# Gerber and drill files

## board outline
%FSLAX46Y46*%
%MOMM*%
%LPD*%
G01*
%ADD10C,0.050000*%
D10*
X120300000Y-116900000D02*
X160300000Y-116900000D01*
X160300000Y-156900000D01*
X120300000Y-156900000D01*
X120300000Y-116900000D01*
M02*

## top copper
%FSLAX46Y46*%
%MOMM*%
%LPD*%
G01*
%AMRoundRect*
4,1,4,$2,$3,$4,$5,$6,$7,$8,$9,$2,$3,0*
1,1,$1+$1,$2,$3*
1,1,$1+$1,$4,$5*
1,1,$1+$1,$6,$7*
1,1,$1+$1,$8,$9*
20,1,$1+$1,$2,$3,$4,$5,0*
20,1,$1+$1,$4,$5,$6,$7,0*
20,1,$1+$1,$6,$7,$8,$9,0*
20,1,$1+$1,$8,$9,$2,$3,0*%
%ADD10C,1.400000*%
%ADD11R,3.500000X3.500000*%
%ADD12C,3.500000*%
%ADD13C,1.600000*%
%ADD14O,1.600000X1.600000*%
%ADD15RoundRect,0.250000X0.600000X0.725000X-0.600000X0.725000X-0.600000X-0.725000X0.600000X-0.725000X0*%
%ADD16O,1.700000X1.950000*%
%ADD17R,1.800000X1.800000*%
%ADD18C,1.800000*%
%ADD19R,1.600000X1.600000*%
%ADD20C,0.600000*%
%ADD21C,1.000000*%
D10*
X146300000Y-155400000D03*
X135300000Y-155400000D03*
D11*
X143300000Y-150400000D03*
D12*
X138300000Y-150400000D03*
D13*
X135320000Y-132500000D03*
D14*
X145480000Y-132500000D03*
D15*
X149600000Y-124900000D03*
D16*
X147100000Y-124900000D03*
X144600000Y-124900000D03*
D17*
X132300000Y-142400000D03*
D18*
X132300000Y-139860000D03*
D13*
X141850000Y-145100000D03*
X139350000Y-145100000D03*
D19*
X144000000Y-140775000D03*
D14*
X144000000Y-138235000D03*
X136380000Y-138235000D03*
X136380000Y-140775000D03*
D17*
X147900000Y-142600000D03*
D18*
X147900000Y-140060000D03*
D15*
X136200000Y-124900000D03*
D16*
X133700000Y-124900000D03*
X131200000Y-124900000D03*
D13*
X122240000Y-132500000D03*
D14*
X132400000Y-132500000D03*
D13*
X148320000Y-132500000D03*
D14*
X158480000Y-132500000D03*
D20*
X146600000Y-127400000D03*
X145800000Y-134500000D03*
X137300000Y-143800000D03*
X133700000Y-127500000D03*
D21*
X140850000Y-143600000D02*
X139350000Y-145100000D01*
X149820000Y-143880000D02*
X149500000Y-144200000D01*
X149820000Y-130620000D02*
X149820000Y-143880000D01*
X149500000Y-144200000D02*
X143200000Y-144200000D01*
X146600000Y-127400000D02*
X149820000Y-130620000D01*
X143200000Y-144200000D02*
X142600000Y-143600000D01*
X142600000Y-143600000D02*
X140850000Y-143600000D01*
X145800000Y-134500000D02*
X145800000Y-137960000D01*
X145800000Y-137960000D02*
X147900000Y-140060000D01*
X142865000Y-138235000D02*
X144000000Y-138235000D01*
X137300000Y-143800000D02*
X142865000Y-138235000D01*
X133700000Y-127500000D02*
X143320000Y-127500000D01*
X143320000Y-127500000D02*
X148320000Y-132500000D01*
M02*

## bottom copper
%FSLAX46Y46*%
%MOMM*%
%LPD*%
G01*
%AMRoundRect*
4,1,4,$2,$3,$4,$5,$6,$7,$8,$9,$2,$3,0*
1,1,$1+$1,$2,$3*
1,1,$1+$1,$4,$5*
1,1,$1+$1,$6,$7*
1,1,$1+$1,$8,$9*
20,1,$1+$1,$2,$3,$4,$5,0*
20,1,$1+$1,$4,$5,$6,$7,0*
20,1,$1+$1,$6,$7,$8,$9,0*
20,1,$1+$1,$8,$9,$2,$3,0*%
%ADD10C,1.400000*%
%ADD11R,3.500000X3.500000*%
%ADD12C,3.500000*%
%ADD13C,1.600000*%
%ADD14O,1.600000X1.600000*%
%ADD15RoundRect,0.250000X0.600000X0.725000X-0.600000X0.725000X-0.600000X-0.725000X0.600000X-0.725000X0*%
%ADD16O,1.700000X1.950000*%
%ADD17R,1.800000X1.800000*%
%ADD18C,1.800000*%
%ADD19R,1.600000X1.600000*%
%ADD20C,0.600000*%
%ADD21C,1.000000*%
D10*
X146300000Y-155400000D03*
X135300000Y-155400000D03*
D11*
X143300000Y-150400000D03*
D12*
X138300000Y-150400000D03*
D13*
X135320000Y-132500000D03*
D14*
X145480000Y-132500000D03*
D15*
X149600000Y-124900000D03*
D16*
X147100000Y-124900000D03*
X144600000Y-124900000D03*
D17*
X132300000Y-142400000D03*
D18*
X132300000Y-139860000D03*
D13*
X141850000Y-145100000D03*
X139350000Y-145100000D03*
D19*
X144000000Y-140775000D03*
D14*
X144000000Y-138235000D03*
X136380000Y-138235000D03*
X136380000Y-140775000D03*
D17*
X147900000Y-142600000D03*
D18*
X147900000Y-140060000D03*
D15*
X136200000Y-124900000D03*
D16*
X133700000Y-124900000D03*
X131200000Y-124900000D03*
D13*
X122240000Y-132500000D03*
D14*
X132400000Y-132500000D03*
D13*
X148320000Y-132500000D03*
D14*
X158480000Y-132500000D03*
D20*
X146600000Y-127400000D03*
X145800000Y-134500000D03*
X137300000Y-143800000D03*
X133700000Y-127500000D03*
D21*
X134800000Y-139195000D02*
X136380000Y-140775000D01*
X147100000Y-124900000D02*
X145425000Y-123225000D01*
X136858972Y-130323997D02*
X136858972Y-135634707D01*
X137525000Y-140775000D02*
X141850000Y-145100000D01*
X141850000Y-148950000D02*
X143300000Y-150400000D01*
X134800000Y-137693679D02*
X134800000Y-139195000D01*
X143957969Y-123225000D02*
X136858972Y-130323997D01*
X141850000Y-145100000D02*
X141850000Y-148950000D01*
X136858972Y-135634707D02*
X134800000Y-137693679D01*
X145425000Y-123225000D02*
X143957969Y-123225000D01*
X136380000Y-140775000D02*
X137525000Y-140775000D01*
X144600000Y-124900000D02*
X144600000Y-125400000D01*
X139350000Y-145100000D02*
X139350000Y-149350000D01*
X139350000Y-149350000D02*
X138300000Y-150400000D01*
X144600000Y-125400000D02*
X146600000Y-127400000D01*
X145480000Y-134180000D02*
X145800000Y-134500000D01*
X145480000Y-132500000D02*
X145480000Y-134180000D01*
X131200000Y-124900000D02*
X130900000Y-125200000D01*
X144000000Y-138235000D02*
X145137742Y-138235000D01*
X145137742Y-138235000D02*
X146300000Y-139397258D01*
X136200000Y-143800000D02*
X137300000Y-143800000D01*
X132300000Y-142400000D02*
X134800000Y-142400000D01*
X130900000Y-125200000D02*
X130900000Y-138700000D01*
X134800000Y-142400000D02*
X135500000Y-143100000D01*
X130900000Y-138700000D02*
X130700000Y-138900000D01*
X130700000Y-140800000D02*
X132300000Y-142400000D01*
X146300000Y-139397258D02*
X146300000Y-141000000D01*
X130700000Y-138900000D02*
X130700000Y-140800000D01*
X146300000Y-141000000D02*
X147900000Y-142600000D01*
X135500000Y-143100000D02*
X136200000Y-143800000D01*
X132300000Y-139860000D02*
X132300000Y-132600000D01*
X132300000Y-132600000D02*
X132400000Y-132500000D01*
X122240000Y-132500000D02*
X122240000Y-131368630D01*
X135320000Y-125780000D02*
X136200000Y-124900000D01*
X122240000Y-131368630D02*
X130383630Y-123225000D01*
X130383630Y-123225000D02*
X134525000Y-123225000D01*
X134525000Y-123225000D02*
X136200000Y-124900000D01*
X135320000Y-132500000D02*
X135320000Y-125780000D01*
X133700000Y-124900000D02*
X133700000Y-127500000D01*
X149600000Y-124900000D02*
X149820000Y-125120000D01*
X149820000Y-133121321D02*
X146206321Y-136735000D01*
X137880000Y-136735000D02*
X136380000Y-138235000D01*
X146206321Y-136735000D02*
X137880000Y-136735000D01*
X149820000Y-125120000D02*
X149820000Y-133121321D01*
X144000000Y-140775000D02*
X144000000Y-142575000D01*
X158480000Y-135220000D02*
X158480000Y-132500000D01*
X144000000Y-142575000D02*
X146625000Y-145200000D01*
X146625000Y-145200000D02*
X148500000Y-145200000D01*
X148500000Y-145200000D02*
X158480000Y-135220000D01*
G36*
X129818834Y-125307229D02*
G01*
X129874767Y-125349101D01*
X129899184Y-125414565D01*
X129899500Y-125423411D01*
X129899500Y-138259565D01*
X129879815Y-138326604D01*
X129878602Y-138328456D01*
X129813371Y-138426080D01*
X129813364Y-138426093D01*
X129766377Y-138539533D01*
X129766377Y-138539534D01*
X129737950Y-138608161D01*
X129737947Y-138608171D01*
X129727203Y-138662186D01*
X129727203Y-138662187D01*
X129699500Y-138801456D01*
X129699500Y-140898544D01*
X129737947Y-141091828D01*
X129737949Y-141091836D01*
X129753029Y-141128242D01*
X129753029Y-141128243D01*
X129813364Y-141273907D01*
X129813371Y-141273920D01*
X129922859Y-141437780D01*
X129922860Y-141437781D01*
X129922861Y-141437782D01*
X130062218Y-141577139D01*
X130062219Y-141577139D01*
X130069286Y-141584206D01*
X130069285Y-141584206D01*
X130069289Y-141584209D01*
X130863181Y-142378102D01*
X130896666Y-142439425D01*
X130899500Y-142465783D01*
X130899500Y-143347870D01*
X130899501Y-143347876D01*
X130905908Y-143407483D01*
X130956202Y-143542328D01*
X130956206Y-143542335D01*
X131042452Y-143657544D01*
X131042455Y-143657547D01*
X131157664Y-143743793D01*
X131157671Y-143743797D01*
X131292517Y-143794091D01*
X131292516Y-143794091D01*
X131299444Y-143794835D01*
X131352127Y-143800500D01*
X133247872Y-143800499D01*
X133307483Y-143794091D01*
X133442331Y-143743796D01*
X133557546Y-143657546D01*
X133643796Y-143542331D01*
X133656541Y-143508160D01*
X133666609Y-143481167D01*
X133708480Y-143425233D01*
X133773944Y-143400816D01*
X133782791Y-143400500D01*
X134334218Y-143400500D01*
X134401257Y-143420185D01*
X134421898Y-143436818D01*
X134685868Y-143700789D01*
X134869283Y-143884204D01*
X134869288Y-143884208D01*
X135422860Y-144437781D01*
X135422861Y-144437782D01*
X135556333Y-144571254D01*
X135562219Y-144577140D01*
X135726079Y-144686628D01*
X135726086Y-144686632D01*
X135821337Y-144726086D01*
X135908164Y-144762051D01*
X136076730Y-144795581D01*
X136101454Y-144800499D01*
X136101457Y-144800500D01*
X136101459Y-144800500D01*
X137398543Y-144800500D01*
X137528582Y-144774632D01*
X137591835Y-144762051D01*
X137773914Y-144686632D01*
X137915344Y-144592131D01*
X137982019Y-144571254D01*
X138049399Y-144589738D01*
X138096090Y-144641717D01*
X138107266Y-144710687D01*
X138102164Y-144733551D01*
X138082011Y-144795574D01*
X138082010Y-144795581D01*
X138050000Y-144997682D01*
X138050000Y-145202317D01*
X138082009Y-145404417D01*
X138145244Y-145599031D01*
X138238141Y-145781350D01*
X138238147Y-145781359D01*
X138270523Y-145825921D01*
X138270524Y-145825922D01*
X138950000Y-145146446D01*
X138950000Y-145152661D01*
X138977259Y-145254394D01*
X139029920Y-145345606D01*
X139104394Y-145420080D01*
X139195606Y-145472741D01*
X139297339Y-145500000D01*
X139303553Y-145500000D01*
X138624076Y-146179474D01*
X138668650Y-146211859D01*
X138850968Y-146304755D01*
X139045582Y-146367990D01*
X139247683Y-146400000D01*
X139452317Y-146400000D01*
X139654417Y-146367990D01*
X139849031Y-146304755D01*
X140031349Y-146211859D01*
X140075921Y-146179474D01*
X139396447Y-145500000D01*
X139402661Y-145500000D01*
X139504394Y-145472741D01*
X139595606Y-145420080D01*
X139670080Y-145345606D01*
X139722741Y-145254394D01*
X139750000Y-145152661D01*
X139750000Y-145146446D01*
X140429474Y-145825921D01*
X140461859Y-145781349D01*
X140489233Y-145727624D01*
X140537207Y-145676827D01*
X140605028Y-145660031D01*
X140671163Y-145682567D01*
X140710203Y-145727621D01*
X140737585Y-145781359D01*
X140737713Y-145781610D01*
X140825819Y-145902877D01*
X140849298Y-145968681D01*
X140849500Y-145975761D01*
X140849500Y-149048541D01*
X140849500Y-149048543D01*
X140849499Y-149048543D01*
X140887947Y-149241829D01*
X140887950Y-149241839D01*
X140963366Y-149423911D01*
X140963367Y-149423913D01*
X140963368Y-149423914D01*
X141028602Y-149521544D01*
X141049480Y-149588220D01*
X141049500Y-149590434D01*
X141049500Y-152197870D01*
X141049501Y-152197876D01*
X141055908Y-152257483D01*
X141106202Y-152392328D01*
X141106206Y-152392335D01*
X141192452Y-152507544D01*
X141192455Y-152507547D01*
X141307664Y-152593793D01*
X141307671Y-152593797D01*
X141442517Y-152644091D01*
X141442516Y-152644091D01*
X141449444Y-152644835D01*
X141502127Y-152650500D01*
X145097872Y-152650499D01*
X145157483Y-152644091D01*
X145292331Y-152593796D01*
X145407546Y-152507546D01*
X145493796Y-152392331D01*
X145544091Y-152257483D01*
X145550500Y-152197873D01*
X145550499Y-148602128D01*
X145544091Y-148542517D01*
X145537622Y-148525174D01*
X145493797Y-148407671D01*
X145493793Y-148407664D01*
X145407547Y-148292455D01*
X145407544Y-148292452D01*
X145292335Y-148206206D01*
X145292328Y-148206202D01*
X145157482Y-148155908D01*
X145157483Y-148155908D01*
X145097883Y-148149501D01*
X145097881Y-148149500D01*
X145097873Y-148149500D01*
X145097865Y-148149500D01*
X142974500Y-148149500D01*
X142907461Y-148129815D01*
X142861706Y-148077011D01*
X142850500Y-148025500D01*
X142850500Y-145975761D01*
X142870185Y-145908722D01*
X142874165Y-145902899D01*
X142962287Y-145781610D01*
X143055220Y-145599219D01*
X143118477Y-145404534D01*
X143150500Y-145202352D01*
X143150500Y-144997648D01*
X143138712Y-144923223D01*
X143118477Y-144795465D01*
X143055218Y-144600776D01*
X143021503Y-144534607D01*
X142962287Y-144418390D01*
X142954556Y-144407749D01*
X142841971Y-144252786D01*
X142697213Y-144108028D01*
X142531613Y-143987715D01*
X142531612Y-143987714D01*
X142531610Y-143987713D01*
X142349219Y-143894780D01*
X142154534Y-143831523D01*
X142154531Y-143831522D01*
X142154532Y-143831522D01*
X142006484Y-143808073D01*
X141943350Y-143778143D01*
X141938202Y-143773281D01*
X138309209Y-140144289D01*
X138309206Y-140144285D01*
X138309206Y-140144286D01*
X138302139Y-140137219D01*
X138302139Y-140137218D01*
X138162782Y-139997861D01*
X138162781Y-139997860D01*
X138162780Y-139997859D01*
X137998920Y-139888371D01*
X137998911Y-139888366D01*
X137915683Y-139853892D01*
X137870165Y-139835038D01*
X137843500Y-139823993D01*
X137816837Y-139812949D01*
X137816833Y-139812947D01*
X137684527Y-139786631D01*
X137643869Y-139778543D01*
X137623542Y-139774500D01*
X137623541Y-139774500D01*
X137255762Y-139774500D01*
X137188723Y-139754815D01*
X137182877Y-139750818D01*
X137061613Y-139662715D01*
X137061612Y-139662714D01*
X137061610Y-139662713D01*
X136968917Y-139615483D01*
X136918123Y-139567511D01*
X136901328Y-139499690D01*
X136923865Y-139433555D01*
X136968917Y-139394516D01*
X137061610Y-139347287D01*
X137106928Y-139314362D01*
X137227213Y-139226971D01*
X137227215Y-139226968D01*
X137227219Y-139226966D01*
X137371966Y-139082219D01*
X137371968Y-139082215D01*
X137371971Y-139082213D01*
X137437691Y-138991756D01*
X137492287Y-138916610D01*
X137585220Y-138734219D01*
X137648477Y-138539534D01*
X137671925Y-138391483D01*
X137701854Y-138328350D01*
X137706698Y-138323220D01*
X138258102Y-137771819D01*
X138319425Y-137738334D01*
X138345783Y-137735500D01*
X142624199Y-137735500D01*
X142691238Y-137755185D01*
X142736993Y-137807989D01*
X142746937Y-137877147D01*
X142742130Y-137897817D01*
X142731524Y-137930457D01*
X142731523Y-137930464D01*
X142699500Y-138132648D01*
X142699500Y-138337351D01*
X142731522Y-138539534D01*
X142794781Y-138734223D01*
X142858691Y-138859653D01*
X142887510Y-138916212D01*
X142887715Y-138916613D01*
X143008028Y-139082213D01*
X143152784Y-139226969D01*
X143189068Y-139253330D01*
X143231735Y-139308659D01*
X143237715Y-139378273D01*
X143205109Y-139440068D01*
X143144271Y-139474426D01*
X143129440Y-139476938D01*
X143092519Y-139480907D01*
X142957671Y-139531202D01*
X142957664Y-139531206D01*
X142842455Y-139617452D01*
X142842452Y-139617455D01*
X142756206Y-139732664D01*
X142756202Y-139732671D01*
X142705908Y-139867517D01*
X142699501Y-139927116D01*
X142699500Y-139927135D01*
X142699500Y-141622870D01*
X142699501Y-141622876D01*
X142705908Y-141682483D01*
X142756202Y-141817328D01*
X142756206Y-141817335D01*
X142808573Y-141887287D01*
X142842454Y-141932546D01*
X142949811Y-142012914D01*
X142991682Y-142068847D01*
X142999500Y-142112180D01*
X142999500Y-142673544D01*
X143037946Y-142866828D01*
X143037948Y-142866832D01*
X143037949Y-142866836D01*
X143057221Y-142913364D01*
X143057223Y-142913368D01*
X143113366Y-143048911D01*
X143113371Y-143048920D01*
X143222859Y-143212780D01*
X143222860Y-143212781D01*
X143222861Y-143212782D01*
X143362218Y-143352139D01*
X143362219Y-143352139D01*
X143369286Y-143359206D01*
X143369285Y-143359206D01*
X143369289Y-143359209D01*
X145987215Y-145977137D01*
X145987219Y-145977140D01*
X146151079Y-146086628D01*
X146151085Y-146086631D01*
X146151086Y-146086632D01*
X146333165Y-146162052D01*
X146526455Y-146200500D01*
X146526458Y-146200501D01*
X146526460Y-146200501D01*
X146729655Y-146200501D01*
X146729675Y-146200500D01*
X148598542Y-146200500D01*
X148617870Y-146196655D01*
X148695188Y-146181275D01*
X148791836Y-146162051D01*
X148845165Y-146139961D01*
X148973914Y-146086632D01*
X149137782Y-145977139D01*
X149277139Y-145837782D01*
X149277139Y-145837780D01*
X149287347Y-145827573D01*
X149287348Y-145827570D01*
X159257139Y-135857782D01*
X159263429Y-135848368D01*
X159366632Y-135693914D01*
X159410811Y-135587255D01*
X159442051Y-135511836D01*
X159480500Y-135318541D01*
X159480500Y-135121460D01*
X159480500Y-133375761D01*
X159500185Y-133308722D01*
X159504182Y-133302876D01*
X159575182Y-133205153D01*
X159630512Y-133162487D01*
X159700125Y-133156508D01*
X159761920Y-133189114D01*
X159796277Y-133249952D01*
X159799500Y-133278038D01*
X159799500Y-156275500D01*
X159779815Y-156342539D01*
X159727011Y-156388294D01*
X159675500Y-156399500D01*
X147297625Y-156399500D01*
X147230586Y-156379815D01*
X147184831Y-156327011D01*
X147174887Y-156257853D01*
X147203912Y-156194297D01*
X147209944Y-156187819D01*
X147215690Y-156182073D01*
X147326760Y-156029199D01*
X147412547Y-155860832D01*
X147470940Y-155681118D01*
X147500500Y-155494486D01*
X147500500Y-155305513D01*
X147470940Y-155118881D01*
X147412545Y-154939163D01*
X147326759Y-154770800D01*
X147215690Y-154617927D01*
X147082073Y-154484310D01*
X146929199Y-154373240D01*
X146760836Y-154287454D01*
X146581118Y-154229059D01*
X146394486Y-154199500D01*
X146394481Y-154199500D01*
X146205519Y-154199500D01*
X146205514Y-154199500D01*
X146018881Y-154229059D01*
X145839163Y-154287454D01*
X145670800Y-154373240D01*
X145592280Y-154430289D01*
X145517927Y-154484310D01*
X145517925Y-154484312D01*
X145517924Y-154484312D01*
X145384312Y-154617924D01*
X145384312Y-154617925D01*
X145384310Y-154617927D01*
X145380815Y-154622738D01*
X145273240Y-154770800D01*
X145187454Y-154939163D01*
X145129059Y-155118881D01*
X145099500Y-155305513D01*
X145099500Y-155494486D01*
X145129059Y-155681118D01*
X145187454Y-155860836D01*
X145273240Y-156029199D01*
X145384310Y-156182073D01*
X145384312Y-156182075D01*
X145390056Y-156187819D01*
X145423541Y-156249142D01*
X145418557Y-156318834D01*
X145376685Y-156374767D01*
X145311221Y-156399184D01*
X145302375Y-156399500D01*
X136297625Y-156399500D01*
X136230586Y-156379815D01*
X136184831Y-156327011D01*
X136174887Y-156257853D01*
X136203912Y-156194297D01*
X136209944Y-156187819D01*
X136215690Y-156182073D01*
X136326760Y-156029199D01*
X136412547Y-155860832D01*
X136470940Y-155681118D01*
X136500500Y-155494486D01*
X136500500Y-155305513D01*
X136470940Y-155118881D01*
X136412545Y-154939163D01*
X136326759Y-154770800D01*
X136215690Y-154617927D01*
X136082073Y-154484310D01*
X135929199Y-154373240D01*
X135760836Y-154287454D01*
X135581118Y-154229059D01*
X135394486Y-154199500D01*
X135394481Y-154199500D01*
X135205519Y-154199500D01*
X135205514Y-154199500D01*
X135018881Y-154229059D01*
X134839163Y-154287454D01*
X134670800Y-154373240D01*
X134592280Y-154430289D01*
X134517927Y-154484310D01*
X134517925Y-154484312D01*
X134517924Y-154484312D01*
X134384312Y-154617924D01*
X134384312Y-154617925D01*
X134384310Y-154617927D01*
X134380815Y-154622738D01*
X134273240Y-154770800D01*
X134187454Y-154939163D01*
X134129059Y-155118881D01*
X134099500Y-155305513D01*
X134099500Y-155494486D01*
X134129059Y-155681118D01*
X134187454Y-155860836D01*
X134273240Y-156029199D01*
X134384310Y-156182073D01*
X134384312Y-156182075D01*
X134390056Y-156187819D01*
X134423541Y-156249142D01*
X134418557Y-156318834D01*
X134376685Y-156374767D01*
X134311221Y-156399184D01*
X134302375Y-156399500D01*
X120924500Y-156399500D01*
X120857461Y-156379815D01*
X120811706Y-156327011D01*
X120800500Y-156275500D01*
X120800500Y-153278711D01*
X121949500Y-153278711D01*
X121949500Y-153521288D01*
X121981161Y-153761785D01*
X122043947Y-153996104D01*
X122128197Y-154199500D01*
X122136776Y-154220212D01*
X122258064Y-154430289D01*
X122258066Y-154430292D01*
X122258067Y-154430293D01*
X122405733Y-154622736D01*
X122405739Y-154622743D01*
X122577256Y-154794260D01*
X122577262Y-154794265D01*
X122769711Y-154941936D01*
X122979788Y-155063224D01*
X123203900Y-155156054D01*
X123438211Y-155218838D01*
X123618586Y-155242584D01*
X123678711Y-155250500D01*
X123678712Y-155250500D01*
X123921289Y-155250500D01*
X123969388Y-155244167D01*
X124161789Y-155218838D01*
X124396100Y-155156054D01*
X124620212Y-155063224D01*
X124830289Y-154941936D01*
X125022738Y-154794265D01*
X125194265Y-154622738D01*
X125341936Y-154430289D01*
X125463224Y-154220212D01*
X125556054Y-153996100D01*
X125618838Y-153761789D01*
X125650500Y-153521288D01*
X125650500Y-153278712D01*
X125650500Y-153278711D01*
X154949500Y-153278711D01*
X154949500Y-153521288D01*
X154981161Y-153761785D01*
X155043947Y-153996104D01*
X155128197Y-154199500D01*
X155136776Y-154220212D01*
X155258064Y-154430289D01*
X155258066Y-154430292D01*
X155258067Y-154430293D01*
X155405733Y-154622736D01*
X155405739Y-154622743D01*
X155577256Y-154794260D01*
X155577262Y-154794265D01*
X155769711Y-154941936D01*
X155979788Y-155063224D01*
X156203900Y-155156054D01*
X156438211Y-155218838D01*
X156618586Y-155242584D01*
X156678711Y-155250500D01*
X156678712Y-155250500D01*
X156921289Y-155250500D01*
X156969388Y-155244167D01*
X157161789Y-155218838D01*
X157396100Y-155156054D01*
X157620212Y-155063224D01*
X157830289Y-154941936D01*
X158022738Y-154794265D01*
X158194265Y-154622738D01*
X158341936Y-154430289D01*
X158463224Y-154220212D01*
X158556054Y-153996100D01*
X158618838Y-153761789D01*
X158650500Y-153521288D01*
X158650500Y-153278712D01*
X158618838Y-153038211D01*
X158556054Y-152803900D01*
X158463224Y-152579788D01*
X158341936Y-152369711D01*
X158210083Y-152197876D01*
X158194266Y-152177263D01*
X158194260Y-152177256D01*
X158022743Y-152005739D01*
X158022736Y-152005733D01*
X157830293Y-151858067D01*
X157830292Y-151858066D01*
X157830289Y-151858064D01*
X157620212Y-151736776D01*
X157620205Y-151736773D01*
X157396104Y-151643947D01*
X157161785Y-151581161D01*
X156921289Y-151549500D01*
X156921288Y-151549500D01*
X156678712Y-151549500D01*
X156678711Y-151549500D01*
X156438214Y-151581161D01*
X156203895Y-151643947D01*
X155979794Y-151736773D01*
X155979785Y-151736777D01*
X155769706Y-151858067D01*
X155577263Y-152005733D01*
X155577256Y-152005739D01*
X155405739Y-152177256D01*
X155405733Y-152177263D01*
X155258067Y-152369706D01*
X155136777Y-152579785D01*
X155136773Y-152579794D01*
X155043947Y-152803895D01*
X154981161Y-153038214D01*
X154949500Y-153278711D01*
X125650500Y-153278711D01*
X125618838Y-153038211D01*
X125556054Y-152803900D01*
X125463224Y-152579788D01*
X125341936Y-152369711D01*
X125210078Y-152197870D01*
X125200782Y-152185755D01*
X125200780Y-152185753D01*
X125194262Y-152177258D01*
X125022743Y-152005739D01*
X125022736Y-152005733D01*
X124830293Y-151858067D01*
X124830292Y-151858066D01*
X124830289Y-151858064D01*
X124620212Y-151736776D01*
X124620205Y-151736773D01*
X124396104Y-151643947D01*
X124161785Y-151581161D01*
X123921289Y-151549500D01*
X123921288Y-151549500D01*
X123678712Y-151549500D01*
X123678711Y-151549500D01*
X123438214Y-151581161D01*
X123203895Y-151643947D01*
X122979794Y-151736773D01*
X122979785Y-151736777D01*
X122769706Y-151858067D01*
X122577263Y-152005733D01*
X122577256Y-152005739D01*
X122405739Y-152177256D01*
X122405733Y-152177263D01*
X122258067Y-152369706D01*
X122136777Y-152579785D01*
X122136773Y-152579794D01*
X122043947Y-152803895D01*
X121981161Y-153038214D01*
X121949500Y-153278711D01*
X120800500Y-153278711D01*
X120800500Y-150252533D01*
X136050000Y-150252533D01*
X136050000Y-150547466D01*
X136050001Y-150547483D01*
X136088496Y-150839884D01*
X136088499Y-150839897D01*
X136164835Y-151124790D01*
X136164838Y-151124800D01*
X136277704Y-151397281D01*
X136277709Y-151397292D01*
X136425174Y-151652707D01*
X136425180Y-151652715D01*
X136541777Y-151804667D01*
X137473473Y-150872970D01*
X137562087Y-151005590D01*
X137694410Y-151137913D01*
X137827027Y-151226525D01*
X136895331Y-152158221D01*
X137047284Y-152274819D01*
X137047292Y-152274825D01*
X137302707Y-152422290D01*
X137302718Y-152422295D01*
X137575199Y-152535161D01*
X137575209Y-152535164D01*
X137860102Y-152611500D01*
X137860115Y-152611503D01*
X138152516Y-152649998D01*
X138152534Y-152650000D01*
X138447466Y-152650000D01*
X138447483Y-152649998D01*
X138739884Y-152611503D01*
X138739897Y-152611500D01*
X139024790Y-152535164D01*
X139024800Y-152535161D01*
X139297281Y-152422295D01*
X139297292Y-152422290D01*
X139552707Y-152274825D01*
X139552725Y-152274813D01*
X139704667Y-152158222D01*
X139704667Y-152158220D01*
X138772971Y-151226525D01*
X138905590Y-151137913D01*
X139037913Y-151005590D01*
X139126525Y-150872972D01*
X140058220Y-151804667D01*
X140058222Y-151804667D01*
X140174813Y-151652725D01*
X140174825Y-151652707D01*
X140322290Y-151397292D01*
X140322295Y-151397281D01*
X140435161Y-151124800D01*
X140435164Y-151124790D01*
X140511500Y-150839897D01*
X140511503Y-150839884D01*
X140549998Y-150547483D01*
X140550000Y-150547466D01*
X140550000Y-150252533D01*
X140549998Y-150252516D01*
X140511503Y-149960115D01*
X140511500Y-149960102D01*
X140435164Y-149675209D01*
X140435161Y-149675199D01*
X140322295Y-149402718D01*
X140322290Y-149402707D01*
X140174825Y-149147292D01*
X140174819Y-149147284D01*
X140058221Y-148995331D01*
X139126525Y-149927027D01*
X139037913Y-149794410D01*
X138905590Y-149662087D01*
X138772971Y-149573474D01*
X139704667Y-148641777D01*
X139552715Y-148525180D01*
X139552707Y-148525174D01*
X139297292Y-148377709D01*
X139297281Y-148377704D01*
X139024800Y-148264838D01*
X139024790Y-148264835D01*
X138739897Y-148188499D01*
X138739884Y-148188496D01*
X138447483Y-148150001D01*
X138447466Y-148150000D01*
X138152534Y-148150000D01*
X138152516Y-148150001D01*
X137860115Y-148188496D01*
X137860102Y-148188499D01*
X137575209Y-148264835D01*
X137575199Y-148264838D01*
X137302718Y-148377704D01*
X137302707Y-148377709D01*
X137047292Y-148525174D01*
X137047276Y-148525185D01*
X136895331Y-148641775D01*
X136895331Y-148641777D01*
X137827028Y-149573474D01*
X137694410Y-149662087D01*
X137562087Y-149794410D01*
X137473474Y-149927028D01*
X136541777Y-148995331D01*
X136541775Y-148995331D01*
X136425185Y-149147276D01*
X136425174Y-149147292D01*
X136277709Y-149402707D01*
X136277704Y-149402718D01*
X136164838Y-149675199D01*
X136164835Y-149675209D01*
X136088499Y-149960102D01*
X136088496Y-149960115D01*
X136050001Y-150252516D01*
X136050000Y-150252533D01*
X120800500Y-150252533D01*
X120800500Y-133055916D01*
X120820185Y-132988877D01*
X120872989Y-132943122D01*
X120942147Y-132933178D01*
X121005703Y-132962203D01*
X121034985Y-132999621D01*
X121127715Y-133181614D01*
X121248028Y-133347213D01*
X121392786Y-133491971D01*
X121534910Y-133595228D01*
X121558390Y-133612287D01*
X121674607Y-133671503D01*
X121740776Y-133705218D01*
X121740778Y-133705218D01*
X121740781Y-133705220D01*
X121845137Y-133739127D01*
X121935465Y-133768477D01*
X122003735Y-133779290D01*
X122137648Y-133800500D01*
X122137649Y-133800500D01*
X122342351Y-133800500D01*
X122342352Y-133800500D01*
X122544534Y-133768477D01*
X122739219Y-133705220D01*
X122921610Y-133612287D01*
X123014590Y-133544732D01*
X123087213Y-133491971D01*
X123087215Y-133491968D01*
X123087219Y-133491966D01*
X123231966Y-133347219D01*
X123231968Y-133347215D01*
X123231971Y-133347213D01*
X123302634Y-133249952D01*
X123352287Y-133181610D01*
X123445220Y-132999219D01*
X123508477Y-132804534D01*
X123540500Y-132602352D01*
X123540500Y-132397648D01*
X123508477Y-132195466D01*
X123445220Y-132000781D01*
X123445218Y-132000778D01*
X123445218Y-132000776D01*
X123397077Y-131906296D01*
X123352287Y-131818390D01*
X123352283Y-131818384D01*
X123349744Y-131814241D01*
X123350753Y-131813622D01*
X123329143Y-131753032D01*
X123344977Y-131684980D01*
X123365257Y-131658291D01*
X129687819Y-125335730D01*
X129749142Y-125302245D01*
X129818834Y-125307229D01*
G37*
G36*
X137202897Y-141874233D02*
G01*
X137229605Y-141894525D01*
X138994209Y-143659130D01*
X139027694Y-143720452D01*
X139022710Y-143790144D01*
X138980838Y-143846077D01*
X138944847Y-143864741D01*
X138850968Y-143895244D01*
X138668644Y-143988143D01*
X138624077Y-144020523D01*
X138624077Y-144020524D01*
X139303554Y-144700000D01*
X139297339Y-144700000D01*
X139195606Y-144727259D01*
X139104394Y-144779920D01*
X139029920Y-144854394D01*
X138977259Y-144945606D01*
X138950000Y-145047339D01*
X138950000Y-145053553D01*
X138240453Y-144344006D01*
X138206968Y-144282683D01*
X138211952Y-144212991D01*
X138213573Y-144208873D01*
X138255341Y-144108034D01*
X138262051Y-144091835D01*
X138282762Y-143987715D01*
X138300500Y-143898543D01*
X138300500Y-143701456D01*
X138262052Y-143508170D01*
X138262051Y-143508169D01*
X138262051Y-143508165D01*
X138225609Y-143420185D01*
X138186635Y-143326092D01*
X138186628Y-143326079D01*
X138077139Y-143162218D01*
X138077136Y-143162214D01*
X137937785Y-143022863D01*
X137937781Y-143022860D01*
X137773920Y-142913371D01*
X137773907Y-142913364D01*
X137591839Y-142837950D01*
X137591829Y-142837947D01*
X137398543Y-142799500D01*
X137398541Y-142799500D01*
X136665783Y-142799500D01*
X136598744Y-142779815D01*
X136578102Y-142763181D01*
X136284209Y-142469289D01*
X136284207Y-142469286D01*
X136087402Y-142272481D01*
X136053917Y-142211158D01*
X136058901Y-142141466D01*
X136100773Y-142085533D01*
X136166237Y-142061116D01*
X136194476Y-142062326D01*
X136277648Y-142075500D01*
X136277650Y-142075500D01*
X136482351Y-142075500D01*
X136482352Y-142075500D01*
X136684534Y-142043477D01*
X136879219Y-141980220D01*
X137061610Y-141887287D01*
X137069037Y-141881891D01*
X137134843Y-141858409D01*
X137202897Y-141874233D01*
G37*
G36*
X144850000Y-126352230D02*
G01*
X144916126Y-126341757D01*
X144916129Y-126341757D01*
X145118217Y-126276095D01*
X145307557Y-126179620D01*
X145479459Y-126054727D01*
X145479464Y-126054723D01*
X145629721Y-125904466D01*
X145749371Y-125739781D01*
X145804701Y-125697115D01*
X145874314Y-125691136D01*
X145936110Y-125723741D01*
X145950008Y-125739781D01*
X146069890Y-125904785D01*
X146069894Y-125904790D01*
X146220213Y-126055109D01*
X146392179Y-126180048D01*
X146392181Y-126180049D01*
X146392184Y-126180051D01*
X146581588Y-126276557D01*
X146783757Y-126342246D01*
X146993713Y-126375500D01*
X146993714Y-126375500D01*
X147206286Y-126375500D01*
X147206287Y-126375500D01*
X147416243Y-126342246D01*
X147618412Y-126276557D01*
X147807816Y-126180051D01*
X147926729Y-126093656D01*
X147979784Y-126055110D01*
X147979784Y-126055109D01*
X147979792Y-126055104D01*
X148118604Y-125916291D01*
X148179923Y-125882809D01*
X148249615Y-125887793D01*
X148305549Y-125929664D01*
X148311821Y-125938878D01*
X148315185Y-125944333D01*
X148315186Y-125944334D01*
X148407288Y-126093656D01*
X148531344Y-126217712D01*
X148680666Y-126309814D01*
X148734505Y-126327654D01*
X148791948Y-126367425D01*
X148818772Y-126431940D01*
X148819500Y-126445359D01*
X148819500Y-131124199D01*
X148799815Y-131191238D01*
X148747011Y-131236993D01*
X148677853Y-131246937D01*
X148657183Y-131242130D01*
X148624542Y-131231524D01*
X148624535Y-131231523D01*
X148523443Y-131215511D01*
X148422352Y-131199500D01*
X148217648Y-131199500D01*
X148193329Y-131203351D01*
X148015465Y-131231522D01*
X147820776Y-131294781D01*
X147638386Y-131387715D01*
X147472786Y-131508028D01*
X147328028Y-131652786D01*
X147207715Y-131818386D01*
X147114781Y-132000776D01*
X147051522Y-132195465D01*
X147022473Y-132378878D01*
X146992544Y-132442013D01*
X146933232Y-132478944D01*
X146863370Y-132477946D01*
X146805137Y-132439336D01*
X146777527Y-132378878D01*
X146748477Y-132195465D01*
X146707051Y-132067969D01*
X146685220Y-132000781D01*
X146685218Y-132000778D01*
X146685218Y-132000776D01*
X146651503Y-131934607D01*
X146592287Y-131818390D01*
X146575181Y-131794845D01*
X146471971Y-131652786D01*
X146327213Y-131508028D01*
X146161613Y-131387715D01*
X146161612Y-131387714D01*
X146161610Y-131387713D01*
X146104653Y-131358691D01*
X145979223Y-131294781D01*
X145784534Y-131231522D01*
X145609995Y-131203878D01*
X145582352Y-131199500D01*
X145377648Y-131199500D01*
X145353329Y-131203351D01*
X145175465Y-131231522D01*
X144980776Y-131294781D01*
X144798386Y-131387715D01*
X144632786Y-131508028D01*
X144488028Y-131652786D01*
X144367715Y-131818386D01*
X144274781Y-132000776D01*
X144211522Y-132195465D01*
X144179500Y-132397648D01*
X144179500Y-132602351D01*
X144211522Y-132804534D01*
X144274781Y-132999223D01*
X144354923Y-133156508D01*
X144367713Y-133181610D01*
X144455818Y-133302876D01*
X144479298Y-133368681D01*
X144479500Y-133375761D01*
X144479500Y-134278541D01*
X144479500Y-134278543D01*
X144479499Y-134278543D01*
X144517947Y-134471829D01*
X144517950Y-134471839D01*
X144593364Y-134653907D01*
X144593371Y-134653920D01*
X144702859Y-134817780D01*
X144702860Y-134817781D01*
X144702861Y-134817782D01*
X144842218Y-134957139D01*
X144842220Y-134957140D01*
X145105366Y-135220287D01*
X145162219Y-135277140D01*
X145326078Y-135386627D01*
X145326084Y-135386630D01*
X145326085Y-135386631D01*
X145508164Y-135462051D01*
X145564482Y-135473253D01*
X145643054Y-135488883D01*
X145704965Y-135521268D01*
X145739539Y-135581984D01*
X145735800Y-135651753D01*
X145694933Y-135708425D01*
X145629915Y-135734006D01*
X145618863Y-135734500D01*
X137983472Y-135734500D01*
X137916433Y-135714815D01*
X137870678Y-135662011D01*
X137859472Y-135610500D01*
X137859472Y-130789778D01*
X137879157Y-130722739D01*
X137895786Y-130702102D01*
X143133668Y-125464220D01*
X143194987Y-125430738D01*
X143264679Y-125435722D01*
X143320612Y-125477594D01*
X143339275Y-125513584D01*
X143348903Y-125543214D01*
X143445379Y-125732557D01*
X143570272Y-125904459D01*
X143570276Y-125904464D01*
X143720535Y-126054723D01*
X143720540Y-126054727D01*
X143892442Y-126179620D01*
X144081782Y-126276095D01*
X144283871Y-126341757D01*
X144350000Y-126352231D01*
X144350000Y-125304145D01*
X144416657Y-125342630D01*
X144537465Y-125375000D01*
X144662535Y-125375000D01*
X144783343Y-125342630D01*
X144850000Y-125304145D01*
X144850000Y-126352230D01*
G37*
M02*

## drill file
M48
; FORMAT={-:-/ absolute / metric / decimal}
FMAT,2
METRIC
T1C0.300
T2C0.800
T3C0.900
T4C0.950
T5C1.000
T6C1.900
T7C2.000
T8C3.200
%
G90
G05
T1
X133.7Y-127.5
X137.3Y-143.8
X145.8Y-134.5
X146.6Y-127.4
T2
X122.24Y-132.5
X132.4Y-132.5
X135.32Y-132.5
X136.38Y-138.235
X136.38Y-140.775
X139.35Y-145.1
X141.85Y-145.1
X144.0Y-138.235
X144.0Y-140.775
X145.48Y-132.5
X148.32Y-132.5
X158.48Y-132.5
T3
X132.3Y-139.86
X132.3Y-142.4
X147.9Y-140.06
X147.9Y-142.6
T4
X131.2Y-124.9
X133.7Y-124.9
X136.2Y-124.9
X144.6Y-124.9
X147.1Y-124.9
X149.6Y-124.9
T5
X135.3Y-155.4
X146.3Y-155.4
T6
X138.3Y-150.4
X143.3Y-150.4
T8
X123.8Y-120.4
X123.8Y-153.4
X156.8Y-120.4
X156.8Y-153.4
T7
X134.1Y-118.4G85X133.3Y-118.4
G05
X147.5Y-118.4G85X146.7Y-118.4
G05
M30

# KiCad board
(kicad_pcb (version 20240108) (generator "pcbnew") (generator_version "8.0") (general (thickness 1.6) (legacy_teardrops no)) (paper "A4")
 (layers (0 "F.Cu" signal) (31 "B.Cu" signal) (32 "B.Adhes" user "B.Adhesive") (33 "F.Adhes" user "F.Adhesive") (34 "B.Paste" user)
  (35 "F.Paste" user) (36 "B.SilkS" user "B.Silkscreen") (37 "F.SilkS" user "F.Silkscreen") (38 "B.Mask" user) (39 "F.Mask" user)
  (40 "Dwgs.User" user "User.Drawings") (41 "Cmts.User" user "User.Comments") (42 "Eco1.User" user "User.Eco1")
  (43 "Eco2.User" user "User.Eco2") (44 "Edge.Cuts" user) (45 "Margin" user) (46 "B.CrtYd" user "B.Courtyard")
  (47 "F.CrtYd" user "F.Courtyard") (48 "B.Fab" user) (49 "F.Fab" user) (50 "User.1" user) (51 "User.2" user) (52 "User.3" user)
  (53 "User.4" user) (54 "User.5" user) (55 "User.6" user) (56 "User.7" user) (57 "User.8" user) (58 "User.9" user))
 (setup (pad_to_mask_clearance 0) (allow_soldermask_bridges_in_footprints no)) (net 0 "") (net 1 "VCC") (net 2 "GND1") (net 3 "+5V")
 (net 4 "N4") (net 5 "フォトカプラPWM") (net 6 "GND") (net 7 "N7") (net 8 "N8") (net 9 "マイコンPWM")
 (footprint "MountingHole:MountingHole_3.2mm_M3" (layer "F.Cu") (at 123.8 153.4)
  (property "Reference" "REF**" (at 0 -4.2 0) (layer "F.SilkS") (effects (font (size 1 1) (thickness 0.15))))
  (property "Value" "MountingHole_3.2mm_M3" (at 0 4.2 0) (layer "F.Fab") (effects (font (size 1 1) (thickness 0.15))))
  (pad "" np_thru_hole circle (at 0 0) (size 3.2 3.2) (drill 3.2) (layers "*.Cu" "*.Mask")))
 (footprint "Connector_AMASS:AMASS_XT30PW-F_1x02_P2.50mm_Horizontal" (layer "F.Cu") (at 143.3 150.4 180)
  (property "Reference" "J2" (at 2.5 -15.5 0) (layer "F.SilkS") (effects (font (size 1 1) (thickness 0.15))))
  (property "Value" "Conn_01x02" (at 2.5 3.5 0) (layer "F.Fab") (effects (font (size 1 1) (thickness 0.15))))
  (pad "" thru_hole circle (at -3 -5 270) (size 1.4 1.4) (drill 1) (layers "*.Cu" "*.Mask") (remove_unused_layers no))
  (pad "" thru_hole circle (at 8 -5 180) (size 1.4 1.4) (drill 1) (layers "*.Cu" "*.Mask") (remove_unused_layers no))
  (pad "1" thru_hole rect (at 0 0 180) (size 3.5 3.5) (drill 1.9) (layers "*.Cu" "*.Mask") (remove_unused_layers no) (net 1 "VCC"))
  (pad "2" thru_hole circle (at 5 0 180) (size 3.5 3.5) (drill 1.9) (layers "*.Cu" "*.Mask") (remove_unused_layers no) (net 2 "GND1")))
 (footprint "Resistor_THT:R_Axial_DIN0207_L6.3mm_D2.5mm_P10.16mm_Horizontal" (layer "F.Cu") (at 135.32 132.5)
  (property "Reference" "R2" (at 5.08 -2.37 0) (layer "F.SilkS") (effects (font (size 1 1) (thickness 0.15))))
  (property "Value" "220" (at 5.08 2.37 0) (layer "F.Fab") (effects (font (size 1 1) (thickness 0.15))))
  (pad "1" thru_hole circle (at 0 0) (size 1.6 1.6) (drill 0.8) (layers "*.Cu" "*.Mask") (remove_unused_layers no) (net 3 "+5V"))
  (pad "2" thru_hole oval (at 10.16 0) (size 1.6 1.6) (drill 0.8) (layers "*.Cu" "*.Mask") (remove_unused_layers no) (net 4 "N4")))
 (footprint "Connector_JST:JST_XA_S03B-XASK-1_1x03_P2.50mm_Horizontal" (layer "F.Cu") (at 149.6 124.9 180)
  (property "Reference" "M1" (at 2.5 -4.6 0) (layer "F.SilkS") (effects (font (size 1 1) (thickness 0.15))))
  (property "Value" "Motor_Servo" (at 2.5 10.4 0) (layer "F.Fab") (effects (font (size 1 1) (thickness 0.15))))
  (pad "" np_thru_hole oval (at 2.5 6.5 180) (size 2.8 2) (drill oval 2.8 2) (layers "*.Cu" "*.Mask"))
  (pad "1" thru_hole roundrect (at 0 0 180) (size 1.7 1.95) (drill 0.95) (layers "*.Cu" "*.Mask") (remove_unused_layers no)
   (roundrect_rratio 0.147059) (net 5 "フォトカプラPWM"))
  (pad "2" thru_hole oval (at 2.5 0 180) (size 1.7 1.95) (drill 0.95) (layers "*.Cu" "*.Mask") (remove_unused_layers no) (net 1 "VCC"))
  (pad "3" thru_hole oval (at 5 0 180) (size 1.7 1.95) (drill 0.95) (layers "*.Cu" "*.Mask") (remove_unused_layers no) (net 2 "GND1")))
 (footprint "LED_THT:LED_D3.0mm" (layer "F.Cu") (at 132.3 142.4 90)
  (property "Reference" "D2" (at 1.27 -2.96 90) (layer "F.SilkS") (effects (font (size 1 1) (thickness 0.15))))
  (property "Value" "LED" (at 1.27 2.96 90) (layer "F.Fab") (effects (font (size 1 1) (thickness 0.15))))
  (pad "1" thru_hole rect (at 0 0 90) (size 1.8 1.8) (drill 0.9) (layers "*.Cu" "*.Mask") (remove_unused_layers no) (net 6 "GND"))
  (pad "2" thru_hole circle (at 2.54 0 90) (size 1.8 1.8) (drill 0.9) (layers "*.Cu" "*.Mask") (remove_unused_layers no) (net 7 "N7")))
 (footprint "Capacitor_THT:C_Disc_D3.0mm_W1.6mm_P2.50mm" (layer "F.Cu") (at 141.85 145.1 180)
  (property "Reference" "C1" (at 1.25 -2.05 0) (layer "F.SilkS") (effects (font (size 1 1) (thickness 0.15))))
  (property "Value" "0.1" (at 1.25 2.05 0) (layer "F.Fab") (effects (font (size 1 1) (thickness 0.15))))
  (pad "1" thru_hole circle (at 0 0 180) (size 1.6 1.6) (drill 0.8) (layers "*.Cu" "*.Mask") (remove_unused_layers no) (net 1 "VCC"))
  (pad "2" thru_hole circle (at 2.5 0 180) (size 1.6 1.6) (drill 0.8) (layers "*.Cu" "*.Mask") (remove_unused_layers no) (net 2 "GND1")))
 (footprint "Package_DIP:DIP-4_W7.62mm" (layer "F.Cu") (at 144 140.775 180)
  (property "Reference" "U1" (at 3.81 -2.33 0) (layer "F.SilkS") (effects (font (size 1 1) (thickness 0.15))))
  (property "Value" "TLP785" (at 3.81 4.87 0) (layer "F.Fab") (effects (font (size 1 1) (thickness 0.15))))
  (pad "1" thru_hole rect (at 0 0 180) (size 1.6 1.6) (drill 0.8) (layers "*.Cu" "*.Mask") (remove_unused_layers no) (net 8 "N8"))
  (pad "2" thru_hole oval (at 0 2.54 180) (size 1.6 1.6) (drill 0.8) (layers "*.Cu" "*.Mask") (remove_unused_layers no) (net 6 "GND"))
  (pad "3" thru_hole oval (at 7.62 2.54 180) (size 1.6 1.6) (drill 0.8) (layers "*.Cu" "*.Mask") (remove_unused_layers no)
   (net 5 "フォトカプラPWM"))
  (pad "4" thru_hole oval (at 7.62 0 180) (size 1.6 1.6) (drill 0.8) (layers "*.Cu" "*.Mask") (remove_unused_layers no) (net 1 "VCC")))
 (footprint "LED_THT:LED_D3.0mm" (layer "F.Cu") (at 147.9 142.6 90)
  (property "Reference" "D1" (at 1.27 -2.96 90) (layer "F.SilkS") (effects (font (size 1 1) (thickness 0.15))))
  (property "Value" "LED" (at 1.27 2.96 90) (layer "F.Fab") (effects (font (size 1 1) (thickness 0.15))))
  (pad "1" thru_hole rect (at 0 0 90) (size 1.8 1.8) (drill 0.9) (layers "*.Cu" "*.Mask") (remove_unused_layers no) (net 6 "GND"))
  (pad "2" thru_hole circle (at 2.54 0 90) (size 1.8 1.8) (drill 0.9) (layers "*.Cu" "*.Mask") (remove_unused_layers no) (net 4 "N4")))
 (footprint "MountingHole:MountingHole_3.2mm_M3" (layer "F.Cu") (at 156.8 153.4)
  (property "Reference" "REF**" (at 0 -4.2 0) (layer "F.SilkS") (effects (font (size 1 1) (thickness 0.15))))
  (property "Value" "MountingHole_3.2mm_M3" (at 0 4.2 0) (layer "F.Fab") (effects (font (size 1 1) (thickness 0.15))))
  (pad "" np_thru_hole circle (at 0 0) (size 3.2 3.2) (drill 3.2) (layers "*.Cu" "*.Mask")))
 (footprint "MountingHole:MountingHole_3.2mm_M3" (layer "F.Cu") (at 156.8 120.4)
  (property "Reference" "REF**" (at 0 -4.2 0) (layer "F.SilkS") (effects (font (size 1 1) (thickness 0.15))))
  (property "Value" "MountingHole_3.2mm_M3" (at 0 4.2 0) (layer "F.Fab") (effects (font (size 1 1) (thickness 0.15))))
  (pad "" np_thru_hole circle (at 0 0) (size 3.2 3.2) (drill 3.2) (layers "*.Cu" "*.Mask")))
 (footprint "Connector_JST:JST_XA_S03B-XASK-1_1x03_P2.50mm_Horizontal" (layer "F.Cu") (at 136.2 124.9 180)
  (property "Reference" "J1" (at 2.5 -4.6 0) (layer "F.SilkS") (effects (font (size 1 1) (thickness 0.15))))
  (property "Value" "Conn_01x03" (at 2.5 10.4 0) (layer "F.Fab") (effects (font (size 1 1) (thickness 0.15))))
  (pad "" np_thru_hole oval (at 2.5 6.5 180) (size 2.8 2) (drill oval 2.8 2) (layers "*.Cu" "*.Mask"))
  (pad "1" thru_hole roundrect (at 0 0 180) (size 1.7 1.95) (drill 0.95) (layers "*.Cu" "*.Mask") (remove_unused_layers no)
   (roundrect_rratio 0.147059) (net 3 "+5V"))
  (pad "2" thru_hole oval (at 2.5 0 180) (size 1.7 1.95) (drill 0.95) (layers "*.Cu" "*.Mask") (remove_unused_layers no) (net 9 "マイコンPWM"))
  (pad "3" thru_hole oval (at 5 0 180) (size 1.7 1.95) (drill 0.95) (layers "*.Cu" "*.Mask") (remove_unused_layers no) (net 6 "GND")))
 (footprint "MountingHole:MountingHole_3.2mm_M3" (layer "F.Cu") (at 123.8 120.4)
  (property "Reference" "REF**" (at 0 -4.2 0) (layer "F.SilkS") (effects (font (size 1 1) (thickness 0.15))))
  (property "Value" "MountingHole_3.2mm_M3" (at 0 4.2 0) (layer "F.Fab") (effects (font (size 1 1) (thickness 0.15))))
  (pad "" np_thru_hole circle (at 0 0) (size 3.2 3.2) (drill 3.2) (layers "*.Cu" "*.Mask")))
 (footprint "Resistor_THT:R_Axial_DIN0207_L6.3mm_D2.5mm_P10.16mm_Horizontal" (layer "F.Cu") (at 122.24 132.5)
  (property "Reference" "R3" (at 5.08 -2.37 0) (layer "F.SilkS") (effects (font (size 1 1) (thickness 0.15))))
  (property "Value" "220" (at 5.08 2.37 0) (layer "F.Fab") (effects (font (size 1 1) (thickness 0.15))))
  (pad "1" thru_hole circle (at 0 0) (size 1.6 1.6) (drill 0.8) (layers "*.Cu" "*.Mask") (remove_unused_layers no) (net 3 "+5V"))
  (pad "2" thru_hole oval (at 10.16 0) (size 1.6 1.6) (drill 0.8) (layers "*.Cu" "*.Mask") (remove_unused_layers no) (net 7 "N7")))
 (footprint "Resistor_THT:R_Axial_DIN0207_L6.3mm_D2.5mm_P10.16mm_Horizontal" (layer "F.Cu") (at 148.32 132.5)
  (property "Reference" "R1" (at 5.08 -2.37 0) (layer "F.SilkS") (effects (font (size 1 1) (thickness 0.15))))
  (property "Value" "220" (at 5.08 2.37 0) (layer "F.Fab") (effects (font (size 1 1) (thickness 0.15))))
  (pad "1" thru_hole circle (at 0 0) (size 1.6 1.6) (drill 0.8) (layers "*.Cu" "*.Mask") (remove_unused_layers no) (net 9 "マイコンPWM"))
  (pad "2" thru_hole oval (at 10.16 0) (size 1.6 1.6) (drill 0.8) (layers "*.Cu" "*.Mask") (remove_unused_layers no) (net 8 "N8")))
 (gr_rect (start 120.3 116.9) (end 160.3 156.9) (stroke (width 0.05) (type default)) (fill none) (layer "Edge.Cuts"))
 (segment (start 134.8 139.195) (end 136.38 140.775) (width 1) (layer "B.Cu") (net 1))
 (segment (start 147.1 124.9) (end 145.425 123.225) (width 1) (layer "B.Cu") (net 1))
 (segment (start 136.858972 130.323997) (end 136.858972 135.634707) (width 1) (layer "B.Cu") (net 1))
 (segment (start 137.525 140.775) (end 141.85 145.1) (width 1) (layer "B.Cu") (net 1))
 (segment (start 141.85 148.95) (end 143.3 150.4) (width 1) (layer "B.Cu") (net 1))
 (segment (start 134.8 137.693679) (end 134.8 139.195) (width 1) (layer "B.Cu") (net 1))
 (segment (start 143.957969 123.225) (end 136.858972 130.323997) (width 1) (layer "B.Cu") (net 1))
 (segment (start 141.85 145.1) (end 141.85 148.95) (width 1) (layer "B.Cu") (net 1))
 (segment (start 136.858972 135.634707) (end 134.8 137.693679) (width 1) (layer "B.Cu") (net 1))
 (segment (start 145.425 123.225) (end 143.957969 123.225) (width 1) (layer "B.Cu") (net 1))
 (segment (start 136.38 140.775) (end 137.525 140.775) (width 1) (layer "B.Cu") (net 1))
 (segment (start 140.85 143.6) (end 139.35 145.1) (width 1) (layer "F.Cu") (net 2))
 (segment (start 149.82 143.88) (end 149.5 144.2) (width 1) (layer "F.Cu") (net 2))
 (segment (start 149.82 130.62) (end 149.82 143.88) (width 1) (layer "F.Cu") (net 2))
 (segment (start 149.5 144.2) (end 143.2 144.2) (width 1) (layer "F.Cu") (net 2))
 (segment (start 146.6 127.4) (end 149.82 130.62) (width 1) (layer "F.Cu") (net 2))
 (segment (start 143.2 144.2) (end 142.6 143.6) (width 1) (layer "F.Cu") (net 2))
 (segment (start 142.6 143.6) (end 140.85 143.6) (width 1) (layer "F.Cu") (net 2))
 (via (at 146.6 127.4) (size 0.6) (drill 0.3) (layers "F.Cu" "B.Cu") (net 2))
 (segment (start 144.6 124.9) (end 144.6 125.4) (width 1) (layer "B.Cu") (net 2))
 (segment (start 139.35 145.1) (end 139.35 149.35) (width 1) (layer "B.Cu") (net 2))
 (segment (start 139.35 149.35) (end 138.3 150.4) (width 1) (layer "B.Cu") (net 2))
 (segment (start 144.6 125.4) (end 146.6 127.4) (width 1) (layer "B.Cu") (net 2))
 (segment (start 145.8 134.5) (end 145.8 137.96) (width 1) (layer "F.Cu") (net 4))
 (segment (start 145.8 137.96) (end 147.9 140.06) (width 1) (layer "F.Cu") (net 4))
 (via (at 145.8 134.5) (size 0.6) (drill 0.3) (layers "F.Cu" "B.Cu") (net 4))
 (segment (start 145.48 134.18) (end 145.8 134.5) (width 1) (layer "B.Cu") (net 4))
 (segment (start 145.48 132.5) (end 145.48 134.18) (width 1) (layer "B.Cu") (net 4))
 (segment (start 142.865 138.235) (end 144 138.235) (width 1) (layer "F.Cu") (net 6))
 (segment (start 137.3 143.8) (end 142.865 138.235) (width 1) (layer "F.Cu") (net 6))
 (via (at 137.3 143.8) (size 0.6) (drill 0.3) (layers "F.Cu" "B.Cu") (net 6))
 (segment (start 131.2 124.9) (end 130.9 125.2) (width 1) (layer "B.Cu") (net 6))
 (segment (start 144 138.235) (end 145.137742 138.235) (width 1) (layer "B.Cu") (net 6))
 (segment (start 145.137742 138.235) (end 146.3 139.397258) (width 1) (layer "B.Cu") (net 6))
 (segment (start 136.2 143.8) (end 137.3 143.8) (width 1) (layer "B.Cu") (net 6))
 (segment (start 132.3 142.4) (end 134.8 142.4) (width 1) (layer "B.Cu") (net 6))
 (segment (start 130.9 125.2) (end 130.9 138.7) (width 1) (layer "B.Cu") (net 6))
 (segment (start 134.8 142.4) (end 135.5 143.1) (width 1) (layer "B.Cu") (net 6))
 (segment (start 130.9 138.7) (end 130.7 138.9) (width 1) (layer "B.Cu") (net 6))
 (segment (start 130.7 140.8) (end 132.3 142.4) (width 1) (layer "B.Cu") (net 6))
 (segment (start 146.3 139.397258) (end 146.3 141) (width 1) (layer "B.Cu") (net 6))
 (segment (start 130.7 138.9) (end 130.7 140.8) (width 1) (layer "B.Cu") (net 6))
 (segment (start 146.3 141) (end 147.9 142.6) (width 1) (layer "B.Cu") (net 6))
 (segment (start 135.5 143.1) (end 136.2 143.8) (width 1) (layer "B.Cu") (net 6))
 (segment (start 132.3 139.86) (end 132.3 132.6) (width 1) (layer "B.Cu") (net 7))
 (segment (start 132.3 132.6) (end 132.4 132.5) (width 1) (layer "B.Cu") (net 7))
 (segment (start 122.24 132.5) (end 122.24 131.36863) (width 1) (layer "B.Cu") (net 3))
 (segment (start 135.32 125.78) (end 136.2 124.9) (width 1) (layer "B.Cu") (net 3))
 (segment (start 122.24 131.36863) (end 130.38363 123.225) (width 1) (layer "B.Cu") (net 3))
 (segment (start 130.38363 123.225) (end 134.525 123.225) (width 1) (layer "B.Cu") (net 3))
 (segment (start 134.525 123.225) (end 136.2 124.9) (width 1) (layer "B.Cu") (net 3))
 (segment (start 135.32 132.5) (end 135.32 125.78) (width 1) (layer "B.Cu") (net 3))
 (segment (start 133.7 127.5) (end 143.32 127.5) (width 1) (layer "F.Cu") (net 9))
 (segment (start 143.32 127.5) (end 148.32 132.5) (width 1) (layer "F.Cu") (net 9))
 (via (at 133.7 127.5) (size 0.6) (drill 0.3) (layers "F.Cu" "B.Cu") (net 9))
 (segment (start 133.7 124.9) (end 133.7 127.5) (width 1) (layer "B.Cu") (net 9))
 (segment (start 149.6 124.9) (end 149.82 125.12) (width 1) (layer "B.Cu") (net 5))
 (segment (start 149.82 133.121321) (end 146.206321 136.735) (width 1) (layer "B.Cu") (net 5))
 (segment (start 137.88 136.735) (end 136.38 138.235) (width 1) (layer "B.Cu") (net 5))
 (segment (start 146.206321 136.735) (end 137.88 136.735) (width 1) (layer "B.Cu") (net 5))
 (segment (start 149.82 125.12) (end 149.82 133.121321) (width 1) (layer "B.Cu") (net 5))
 (segment (start 144 140.775) (end 144 142.575) (width 1) (layer "B.Cu") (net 8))
 (segment (start 158.48 135.22) (end 158.48 132.5) (width 1) (layer "B.Cu") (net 8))
 (segment (start 144 142.575) (end 146.625 145.2) (width 1) (layer "B.Cu") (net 8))
 (segment (start 146.625 145.2) (end 148.5 145.2) (width 1) (layer "B.Cu") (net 8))
 (segment (start 148.5 145.2) (end 158.48 135.22) (width 1) (layer "B.Cu") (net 8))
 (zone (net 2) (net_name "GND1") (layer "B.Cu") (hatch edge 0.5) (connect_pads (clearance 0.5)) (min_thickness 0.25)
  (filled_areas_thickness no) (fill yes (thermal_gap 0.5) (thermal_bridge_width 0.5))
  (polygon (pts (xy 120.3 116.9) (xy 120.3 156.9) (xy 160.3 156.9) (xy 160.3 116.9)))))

